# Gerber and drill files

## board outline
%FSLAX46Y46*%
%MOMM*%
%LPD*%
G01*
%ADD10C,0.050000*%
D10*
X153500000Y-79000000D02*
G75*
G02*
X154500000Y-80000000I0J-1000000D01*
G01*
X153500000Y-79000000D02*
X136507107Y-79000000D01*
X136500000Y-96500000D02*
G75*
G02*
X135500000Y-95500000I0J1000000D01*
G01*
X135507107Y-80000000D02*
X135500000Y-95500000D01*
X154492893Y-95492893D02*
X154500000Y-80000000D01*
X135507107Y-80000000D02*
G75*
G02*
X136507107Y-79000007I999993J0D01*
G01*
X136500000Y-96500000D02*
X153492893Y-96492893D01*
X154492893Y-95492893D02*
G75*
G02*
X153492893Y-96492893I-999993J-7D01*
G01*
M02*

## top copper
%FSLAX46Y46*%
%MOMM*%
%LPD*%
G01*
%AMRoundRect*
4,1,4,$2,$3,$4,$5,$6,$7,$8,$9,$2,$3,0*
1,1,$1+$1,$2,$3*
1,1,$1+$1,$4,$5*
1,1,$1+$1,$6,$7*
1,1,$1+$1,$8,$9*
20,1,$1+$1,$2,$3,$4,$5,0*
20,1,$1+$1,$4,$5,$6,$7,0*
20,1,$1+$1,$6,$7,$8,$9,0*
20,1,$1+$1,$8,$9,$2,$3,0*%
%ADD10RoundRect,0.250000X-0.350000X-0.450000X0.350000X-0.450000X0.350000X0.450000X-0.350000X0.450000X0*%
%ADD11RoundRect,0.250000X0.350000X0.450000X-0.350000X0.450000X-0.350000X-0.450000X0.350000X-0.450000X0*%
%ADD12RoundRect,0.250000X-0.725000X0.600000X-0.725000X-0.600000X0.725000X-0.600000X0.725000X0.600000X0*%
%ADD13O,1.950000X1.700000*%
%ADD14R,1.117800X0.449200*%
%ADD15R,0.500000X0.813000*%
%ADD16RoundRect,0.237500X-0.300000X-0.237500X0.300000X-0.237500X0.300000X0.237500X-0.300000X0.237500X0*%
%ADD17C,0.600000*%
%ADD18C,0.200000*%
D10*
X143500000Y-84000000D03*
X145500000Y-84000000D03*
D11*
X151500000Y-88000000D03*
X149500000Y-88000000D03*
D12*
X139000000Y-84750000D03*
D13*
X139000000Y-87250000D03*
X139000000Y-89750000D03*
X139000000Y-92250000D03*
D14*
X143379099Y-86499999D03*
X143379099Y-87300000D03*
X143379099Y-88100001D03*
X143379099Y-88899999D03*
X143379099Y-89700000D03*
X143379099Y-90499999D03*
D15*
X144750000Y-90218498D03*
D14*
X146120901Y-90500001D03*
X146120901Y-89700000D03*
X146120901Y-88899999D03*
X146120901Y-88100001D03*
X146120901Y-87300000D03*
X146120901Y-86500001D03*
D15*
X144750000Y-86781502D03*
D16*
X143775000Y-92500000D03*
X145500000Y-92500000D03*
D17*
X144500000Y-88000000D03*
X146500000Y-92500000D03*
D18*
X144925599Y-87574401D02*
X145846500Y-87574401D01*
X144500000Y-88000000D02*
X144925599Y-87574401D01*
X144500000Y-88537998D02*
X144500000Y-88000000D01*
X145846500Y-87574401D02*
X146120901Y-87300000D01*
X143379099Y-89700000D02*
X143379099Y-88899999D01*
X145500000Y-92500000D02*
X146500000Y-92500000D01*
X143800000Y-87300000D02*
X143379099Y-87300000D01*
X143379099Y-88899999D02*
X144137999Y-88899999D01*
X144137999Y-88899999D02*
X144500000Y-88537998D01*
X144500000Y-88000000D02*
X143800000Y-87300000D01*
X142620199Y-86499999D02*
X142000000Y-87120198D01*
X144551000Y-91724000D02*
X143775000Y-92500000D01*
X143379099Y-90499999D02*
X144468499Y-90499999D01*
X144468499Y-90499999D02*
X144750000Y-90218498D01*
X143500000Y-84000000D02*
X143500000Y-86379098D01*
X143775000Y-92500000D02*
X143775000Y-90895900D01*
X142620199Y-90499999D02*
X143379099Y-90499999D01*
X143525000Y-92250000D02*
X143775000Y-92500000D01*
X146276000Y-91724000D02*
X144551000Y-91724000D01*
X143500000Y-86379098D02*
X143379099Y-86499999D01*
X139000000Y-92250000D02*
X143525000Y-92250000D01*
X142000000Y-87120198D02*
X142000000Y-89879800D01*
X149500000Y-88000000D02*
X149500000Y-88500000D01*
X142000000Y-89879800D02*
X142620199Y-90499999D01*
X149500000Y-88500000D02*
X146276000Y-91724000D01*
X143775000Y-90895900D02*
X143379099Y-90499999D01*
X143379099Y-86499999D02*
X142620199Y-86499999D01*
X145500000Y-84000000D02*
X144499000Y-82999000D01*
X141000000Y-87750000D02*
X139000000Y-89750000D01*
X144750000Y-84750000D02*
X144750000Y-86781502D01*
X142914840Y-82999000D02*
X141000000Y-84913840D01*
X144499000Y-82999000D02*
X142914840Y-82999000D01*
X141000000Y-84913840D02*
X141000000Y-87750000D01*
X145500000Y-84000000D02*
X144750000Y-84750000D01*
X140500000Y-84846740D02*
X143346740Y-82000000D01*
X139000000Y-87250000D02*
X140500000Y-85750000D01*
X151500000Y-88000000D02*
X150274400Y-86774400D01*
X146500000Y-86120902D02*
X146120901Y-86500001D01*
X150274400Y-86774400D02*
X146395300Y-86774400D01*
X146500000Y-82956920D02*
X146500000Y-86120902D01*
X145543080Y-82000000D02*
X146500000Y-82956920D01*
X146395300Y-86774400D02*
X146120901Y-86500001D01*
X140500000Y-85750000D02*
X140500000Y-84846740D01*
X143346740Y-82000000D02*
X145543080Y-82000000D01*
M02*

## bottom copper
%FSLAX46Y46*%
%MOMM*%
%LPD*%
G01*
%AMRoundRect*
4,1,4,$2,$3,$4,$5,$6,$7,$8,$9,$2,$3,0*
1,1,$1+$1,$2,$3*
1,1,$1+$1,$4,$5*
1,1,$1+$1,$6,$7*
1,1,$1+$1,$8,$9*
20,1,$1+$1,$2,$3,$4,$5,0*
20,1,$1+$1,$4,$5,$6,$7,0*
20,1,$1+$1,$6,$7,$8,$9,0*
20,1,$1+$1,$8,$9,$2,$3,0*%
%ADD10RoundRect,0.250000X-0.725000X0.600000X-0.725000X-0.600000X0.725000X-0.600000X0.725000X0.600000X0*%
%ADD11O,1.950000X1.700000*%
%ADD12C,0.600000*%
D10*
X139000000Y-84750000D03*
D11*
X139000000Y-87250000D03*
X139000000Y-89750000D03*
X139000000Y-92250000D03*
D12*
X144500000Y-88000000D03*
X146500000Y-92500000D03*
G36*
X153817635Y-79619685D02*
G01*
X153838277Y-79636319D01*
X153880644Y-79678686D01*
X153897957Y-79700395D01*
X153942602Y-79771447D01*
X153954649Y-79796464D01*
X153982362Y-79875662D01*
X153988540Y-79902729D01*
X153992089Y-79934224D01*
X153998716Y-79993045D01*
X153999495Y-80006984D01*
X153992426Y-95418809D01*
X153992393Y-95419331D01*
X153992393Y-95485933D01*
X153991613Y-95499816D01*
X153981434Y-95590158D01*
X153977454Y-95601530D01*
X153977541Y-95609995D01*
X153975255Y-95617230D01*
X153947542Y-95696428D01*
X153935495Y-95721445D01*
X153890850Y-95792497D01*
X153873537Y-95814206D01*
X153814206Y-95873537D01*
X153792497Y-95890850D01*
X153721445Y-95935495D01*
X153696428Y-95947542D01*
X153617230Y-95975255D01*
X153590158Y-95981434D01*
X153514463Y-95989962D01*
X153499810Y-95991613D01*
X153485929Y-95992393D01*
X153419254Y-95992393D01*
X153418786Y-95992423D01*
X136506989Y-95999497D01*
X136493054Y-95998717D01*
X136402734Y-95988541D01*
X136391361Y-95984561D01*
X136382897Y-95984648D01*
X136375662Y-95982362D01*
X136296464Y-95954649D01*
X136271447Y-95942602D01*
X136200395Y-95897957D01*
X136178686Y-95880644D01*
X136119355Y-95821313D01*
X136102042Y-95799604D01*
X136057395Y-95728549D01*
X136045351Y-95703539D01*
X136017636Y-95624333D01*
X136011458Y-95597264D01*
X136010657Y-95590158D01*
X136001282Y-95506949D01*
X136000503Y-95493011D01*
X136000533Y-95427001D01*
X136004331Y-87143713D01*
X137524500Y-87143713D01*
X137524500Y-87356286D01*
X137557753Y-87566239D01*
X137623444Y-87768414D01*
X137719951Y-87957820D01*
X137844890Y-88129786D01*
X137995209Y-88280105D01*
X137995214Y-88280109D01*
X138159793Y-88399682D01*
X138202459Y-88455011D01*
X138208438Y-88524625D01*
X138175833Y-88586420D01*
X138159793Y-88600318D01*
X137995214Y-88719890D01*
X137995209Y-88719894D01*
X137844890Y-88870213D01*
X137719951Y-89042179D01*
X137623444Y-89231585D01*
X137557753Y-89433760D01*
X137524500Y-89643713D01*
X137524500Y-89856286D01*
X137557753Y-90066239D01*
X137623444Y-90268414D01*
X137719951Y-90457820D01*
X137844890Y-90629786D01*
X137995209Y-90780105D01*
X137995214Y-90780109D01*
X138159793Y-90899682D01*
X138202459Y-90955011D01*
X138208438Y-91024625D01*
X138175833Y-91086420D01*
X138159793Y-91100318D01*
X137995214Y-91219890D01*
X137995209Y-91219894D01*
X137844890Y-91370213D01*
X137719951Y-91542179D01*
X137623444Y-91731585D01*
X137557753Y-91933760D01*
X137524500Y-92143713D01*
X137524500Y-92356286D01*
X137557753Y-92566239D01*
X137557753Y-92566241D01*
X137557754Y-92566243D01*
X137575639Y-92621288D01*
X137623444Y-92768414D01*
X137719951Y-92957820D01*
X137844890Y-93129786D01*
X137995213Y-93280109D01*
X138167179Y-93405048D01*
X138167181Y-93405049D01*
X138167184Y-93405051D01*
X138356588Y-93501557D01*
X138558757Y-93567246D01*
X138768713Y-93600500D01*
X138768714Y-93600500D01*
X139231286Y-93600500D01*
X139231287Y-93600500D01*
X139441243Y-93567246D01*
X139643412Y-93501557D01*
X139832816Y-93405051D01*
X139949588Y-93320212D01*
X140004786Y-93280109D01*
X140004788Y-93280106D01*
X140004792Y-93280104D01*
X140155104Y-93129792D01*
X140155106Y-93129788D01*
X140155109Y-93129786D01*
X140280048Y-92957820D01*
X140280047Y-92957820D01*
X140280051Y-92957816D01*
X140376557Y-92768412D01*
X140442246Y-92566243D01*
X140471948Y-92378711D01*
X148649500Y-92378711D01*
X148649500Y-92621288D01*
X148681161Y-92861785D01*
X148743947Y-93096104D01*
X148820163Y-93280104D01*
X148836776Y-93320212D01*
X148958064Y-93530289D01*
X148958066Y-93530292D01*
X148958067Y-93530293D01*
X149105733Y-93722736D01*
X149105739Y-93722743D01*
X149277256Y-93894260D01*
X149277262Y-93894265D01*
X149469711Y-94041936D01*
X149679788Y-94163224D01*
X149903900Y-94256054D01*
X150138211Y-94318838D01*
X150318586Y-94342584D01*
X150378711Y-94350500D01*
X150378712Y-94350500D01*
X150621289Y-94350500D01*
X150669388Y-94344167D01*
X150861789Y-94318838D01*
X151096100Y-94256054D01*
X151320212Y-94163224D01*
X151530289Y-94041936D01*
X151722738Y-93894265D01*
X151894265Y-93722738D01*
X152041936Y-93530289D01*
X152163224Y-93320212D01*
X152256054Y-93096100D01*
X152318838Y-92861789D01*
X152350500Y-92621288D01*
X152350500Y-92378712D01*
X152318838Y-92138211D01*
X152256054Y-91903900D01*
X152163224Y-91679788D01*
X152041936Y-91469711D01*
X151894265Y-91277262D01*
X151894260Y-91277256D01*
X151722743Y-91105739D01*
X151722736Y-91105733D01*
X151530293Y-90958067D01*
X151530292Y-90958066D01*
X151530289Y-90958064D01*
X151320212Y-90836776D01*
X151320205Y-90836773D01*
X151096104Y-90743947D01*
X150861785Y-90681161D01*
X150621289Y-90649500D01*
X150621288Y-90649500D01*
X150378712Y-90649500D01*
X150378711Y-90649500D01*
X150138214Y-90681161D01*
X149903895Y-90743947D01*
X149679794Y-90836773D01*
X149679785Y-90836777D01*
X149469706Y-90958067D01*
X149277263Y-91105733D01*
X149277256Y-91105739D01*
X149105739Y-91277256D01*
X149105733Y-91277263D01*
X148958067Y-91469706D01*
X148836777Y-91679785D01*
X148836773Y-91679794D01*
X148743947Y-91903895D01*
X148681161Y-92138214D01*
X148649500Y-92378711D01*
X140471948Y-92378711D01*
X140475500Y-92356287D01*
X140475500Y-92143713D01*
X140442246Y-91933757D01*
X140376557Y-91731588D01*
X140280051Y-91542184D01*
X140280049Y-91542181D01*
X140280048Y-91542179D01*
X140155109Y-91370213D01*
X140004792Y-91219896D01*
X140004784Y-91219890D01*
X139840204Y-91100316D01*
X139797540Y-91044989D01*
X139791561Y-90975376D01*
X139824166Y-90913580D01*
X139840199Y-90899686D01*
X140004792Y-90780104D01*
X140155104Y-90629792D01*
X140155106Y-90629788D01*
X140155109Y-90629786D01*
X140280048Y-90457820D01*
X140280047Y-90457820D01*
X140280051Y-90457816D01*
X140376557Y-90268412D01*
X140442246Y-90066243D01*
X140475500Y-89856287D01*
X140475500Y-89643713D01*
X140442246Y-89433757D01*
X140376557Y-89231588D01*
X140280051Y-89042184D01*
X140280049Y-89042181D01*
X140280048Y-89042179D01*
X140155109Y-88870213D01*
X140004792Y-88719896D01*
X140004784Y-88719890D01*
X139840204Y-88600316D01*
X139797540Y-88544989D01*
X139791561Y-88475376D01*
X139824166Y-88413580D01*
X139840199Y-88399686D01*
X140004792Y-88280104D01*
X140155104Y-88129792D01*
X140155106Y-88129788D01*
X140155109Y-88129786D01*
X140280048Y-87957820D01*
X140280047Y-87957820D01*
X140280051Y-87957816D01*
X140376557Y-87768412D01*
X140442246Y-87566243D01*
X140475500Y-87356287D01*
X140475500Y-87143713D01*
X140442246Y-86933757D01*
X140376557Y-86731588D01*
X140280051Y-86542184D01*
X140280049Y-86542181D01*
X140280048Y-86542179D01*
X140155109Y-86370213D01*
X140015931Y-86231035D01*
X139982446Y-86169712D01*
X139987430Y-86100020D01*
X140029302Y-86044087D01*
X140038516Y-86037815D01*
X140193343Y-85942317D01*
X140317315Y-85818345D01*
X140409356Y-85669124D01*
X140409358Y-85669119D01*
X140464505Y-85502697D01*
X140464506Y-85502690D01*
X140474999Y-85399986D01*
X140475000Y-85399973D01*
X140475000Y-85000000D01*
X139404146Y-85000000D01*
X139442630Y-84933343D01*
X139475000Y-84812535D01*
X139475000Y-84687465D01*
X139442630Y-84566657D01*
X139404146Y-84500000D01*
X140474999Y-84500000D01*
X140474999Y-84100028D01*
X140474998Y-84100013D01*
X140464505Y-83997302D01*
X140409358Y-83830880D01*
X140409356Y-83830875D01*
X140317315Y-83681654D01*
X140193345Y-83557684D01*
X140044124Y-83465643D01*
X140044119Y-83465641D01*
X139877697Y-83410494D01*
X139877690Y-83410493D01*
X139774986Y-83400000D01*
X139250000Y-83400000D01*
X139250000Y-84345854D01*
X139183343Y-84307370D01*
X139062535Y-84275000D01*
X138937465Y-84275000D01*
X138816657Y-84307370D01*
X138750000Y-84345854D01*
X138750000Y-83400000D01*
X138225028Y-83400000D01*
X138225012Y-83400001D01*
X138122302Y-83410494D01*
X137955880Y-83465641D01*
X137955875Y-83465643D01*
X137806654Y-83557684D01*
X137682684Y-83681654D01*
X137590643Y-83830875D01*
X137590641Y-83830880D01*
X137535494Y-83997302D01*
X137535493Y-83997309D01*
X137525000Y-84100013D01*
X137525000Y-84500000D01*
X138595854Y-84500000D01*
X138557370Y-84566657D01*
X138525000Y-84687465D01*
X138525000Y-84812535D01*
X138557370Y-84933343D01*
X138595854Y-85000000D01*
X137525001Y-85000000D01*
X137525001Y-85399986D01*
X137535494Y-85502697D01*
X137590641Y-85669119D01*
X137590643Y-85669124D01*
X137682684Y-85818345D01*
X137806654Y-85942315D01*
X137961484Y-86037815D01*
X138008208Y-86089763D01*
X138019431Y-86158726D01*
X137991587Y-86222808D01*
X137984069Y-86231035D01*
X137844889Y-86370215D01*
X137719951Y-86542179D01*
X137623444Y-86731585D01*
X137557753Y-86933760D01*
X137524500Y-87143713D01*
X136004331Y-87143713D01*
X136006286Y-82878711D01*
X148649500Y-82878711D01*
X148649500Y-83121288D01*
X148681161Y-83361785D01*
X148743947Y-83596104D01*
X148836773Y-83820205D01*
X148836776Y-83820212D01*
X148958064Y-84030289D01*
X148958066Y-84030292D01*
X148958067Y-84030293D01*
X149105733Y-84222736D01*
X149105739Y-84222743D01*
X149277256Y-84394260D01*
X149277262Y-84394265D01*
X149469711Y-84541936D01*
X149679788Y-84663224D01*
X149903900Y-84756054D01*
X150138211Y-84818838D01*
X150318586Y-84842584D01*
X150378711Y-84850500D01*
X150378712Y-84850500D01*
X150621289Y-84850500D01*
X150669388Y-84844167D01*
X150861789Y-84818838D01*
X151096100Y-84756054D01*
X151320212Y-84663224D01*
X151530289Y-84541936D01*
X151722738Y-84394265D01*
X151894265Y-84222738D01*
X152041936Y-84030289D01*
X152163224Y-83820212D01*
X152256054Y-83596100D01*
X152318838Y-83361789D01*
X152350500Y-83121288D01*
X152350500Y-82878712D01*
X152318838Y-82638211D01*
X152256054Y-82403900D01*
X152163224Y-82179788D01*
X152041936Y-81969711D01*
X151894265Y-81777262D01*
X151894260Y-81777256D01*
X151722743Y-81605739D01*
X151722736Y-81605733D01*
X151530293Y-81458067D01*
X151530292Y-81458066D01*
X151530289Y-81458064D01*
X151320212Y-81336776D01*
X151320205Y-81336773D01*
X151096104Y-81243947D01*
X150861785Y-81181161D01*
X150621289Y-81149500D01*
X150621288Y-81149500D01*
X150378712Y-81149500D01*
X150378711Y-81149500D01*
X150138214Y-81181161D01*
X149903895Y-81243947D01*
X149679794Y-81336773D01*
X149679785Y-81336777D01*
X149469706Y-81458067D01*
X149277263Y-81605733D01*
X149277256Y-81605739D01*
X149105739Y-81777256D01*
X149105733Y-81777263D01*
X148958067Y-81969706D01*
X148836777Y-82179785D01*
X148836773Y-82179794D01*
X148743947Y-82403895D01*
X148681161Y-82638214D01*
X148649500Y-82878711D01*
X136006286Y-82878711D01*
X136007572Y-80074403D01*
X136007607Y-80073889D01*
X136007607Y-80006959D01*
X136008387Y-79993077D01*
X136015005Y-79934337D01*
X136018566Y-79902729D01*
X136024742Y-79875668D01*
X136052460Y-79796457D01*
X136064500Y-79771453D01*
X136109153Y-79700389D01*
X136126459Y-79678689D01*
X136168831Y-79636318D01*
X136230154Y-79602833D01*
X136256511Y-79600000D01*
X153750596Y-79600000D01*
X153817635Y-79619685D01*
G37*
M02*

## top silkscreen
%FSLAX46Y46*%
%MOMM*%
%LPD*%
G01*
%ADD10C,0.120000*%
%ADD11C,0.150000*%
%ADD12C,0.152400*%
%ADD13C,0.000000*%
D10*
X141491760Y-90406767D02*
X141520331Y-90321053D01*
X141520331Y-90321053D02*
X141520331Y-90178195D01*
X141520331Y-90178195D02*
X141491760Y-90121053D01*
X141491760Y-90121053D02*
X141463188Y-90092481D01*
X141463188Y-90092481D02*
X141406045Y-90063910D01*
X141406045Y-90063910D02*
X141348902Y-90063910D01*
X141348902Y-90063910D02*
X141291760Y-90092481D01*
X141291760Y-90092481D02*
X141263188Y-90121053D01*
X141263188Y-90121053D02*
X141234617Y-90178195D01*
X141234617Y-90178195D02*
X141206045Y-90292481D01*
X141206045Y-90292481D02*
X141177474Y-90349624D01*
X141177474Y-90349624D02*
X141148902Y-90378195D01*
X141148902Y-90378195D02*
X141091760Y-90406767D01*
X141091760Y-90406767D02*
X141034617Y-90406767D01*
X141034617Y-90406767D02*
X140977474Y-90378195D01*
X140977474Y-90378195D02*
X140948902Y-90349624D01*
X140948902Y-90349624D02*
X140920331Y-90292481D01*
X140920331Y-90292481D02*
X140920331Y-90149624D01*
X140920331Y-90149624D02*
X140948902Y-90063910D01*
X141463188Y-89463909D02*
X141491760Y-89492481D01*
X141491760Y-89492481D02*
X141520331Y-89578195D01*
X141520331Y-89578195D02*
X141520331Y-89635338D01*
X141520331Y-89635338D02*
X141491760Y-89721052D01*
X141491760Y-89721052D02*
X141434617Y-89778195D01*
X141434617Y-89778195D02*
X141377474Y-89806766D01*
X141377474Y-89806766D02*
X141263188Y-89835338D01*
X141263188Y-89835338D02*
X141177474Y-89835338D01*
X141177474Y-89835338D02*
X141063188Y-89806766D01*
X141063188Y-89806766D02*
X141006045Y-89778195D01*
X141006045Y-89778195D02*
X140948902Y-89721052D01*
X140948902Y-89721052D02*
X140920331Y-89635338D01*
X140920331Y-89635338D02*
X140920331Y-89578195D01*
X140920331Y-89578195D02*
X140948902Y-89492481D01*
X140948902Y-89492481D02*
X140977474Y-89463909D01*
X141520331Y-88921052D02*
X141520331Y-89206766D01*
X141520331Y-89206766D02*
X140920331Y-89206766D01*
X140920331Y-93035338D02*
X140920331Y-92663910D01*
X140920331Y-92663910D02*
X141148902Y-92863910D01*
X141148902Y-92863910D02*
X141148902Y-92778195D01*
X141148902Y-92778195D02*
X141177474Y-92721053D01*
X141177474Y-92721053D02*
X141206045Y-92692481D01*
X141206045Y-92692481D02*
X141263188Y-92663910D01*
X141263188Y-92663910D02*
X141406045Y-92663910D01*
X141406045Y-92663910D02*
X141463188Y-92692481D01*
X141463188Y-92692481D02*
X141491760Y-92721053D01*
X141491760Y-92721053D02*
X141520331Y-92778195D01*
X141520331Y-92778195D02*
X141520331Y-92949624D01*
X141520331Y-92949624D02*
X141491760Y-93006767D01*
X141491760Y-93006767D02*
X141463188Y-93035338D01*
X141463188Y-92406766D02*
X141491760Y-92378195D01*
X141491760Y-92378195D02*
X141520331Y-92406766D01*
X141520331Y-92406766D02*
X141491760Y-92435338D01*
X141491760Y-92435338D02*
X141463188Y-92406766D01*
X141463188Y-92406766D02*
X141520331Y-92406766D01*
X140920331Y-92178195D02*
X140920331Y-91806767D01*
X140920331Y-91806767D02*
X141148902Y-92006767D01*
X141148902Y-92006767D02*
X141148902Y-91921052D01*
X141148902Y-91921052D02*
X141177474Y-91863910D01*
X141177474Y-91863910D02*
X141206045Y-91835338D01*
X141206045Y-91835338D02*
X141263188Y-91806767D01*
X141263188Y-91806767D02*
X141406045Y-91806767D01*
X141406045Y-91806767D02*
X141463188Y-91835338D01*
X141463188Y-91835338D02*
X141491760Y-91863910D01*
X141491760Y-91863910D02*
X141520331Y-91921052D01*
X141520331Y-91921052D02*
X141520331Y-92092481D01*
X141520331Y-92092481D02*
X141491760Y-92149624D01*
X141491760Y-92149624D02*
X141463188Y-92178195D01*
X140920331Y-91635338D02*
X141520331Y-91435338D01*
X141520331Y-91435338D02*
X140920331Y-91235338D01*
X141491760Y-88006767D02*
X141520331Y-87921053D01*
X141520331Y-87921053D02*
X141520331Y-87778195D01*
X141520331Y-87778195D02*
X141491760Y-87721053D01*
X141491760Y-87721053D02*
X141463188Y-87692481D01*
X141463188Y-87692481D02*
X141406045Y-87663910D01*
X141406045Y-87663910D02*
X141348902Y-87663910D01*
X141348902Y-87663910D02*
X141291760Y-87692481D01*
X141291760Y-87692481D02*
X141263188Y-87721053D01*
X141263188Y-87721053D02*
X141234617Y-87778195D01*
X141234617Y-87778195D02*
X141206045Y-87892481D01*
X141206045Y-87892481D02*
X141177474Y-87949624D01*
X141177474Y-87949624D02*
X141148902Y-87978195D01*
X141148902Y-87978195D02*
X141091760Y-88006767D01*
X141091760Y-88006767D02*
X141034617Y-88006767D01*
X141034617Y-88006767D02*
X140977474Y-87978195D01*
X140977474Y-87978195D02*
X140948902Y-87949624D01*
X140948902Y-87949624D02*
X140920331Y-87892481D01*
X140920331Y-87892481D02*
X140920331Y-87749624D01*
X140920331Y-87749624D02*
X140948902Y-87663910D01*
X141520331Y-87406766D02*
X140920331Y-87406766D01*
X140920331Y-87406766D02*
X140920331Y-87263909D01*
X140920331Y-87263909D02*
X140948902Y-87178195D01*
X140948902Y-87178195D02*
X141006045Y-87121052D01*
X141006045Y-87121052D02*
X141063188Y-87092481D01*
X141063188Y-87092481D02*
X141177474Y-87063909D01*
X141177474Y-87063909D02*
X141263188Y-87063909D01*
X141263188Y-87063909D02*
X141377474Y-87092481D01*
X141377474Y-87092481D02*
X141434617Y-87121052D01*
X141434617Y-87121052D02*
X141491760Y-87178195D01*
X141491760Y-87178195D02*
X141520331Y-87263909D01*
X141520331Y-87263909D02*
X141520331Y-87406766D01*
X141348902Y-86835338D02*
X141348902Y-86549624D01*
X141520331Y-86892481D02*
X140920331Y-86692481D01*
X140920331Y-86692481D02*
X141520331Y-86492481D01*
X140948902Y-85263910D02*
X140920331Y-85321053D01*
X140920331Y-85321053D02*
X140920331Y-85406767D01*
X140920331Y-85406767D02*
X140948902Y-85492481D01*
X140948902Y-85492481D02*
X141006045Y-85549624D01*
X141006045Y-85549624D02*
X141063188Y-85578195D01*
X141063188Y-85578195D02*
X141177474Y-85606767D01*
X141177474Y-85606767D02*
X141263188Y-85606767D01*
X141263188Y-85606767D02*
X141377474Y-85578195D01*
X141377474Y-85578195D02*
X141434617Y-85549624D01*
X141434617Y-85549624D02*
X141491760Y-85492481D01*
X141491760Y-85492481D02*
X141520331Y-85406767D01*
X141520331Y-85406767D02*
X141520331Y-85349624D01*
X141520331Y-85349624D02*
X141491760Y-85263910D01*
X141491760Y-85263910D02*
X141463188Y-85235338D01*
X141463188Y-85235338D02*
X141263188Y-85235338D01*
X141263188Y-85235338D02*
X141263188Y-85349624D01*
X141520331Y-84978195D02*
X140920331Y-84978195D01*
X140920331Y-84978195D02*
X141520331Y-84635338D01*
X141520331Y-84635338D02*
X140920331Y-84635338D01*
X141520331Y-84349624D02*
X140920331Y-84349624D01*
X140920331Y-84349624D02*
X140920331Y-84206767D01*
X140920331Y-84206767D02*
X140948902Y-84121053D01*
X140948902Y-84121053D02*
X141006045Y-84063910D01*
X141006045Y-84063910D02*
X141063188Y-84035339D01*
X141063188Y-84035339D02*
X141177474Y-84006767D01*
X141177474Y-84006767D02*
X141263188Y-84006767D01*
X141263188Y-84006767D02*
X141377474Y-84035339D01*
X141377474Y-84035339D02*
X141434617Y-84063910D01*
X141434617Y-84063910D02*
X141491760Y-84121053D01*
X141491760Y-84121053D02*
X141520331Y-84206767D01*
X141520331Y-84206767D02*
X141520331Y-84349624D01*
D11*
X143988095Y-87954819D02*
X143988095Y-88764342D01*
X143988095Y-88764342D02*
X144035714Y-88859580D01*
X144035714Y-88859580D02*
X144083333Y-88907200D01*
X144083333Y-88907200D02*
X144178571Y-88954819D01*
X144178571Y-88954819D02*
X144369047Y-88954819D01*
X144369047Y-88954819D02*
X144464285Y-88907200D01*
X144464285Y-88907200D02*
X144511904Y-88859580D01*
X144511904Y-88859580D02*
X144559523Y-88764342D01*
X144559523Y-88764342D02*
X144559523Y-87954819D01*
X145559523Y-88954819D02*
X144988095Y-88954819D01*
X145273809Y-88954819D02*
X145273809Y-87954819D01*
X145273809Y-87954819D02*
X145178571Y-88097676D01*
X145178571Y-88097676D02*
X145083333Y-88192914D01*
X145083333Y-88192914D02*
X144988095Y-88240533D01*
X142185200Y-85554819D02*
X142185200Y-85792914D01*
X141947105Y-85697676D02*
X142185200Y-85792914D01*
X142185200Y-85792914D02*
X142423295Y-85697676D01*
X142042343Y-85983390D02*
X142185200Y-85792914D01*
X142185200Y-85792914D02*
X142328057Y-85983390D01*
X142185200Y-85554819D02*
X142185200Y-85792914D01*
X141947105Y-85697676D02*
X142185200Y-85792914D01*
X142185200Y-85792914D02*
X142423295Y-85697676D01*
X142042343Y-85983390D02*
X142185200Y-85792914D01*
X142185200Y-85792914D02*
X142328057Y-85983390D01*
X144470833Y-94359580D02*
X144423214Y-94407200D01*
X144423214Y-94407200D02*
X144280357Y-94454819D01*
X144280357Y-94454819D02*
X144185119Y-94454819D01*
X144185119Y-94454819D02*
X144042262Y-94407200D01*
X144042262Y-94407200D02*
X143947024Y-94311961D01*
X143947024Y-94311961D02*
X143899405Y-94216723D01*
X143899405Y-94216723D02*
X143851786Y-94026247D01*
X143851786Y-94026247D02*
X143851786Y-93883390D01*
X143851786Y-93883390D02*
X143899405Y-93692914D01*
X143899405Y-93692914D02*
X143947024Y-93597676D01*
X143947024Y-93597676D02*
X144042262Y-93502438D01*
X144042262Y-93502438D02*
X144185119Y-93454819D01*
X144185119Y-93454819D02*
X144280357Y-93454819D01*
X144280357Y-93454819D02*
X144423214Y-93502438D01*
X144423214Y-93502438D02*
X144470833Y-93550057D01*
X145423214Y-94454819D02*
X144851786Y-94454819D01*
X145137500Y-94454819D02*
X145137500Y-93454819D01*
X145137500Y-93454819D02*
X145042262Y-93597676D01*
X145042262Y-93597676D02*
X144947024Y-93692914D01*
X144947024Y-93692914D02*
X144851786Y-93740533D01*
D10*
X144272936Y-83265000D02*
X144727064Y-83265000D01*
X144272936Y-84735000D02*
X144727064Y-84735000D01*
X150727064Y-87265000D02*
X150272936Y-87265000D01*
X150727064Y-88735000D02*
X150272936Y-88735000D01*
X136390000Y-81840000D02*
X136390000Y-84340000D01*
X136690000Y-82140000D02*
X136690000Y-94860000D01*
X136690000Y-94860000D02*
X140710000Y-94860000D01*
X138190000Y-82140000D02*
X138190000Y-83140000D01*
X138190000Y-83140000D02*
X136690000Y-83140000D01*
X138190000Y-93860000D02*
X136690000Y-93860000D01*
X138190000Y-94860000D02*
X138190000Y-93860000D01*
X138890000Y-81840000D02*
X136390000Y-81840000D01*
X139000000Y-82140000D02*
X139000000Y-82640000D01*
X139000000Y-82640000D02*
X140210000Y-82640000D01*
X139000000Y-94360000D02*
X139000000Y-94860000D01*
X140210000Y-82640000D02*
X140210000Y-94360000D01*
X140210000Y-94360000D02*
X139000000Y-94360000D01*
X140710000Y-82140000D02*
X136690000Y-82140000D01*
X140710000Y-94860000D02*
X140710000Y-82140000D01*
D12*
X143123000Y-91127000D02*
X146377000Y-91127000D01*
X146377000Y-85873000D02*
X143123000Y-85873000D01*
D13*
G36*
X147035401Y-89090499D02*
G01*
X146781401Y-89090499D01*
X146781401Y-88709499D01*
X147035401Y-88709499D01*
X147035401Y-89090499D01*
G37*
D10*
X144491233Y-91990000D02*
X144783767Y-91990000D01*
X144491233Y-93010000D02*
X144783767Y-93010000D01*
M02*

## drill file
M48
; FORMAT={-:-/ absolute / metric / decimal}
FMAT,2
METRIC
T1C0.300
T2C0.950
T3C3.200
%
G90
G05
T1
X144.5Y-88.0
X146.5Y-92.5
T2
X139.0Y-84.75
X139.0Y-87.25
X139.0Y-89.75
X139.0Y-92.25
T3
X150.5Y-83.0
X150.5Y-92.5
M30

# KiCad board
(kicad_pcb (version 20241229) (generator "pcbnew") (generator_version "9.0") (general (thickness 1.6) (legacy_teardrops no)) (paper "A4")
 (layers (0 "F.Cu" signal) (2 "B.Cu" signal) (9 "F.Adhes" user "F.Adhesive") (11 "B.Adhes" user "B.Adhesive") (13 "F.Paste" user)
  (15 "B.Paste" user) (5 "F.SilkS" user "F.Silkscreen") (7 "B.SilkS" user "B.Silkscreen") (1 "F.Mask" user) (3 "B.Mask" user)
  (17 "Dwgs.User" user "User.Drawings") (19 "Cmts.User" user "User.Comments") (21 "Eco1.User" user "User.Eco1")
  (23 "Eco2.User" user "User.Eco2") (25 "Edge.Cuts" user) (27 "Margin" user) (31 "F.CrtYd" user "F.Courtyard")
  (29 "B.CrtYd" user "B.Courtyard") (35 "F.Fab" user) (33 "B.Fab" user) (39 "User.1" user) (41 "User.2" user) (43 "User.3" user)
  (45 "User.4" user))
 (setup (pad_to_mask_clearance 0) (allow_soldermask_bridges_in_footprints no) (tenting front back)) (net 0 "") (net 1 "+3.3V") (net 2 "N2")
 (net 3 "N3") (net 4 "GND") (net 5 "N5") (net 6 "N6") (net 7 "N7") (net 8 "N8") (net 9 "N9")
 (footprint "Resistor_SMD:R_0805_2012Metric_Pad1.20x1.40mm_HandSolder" (layer "F.Cu") (at 144.5 84)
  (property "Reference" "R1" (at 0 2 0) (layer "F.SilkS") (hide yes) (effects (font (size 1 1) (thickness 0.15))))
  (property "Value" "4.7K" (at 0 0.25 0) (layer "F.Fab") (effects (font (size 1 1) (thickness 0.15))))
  (fp_line (start -0.227064 -0.735) (end 0.227064 -0.735) (stroke (width 0.12) (type solid)) (layer "F.SilkS"))
  (fp_line (start -0.227064 0.735) (end 0.227064 0.735) (stroke (width 0.12) (type solid)) (layer "F.SilkS"))
  (pad "1" smd roundrect (at -1 0) (size 1.2 1.4) (layers "F.Cu" "F.Mask" "F.Paste") (roundrect_rratio 0.208333) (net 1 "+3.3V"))
  (pad "2" smd roundrect (at 1 0) (size 1.2 1.4) (layers "F.Cu" "F.Mask" "F.Paste") (roundrect_rratio 0.208333) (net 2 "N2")))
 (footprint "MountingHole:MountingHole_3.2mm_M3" (layer "F.Cu") (at 150.5 83)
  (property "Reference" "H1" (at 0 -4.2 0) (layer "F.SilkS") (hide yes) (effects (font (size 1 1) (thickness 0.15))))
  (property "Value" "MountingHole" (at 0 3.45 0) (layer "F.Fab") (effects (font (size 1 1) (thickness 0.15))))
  (pad "" np_thru_hole circle (at 0 0) (size 3.2 3.2) (drill 3.2) (layers "*.Cu" "*.Mask")))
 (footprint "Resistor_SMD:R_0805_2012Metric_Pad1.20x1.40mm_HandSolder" (layer "F.Cu") (at 150.5 88 180)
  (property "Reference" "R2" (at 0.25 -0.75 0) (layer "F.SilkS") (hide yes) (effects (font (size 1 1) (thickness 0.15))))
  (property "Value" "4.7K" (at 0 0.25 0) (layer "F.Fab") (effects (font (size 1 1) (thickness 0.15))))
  (fp_line (start -0.227064 0.735) (end 0.227064 0.735) (stroke (width 0.12) (type solid)) (layer "F.SilkS"))
  (fp_line (start -0.227064 -0.735) (end 0.227064 -0.735) (stroke (width 0.12) (type solid)) (layer "F.SilkS"))
  (pad "1" smd roundrect (at -1 0 180) (size 1.2 1.4) (layers "F.Cu" "F.Mask" "F.Paste") (roundrect_rratio 0.208333) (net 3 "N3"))
  (pad "2" smd roundrect (at 1 0 180) (size 1.2 1.4) (layers "F.Cu" "F.Mask" "F.Paste") (roundrect_rratio 0.208333) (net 1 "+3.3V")))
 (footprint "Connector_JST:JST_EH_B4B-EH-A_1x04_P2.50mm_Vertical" (layer "F.Cu") (at 139 84.75 -90)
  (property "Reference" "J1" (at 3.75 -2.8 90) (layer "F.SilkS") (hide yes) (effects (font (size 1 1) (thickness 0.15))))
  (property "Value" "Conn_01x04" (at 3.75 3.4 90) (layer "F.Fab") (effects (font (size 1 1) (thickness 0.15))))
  (fp_line (start -2.91 2.61) (end -0.41 2.61) (stroke (width 0.12) (type solid)) (layer "F.SilkS"))
  (fp_line (start -2.61 2.31) (end 10.11 2.31) (stroke (width 0.12) (type solid)) (layer "F.SilkS"))
  (fp_line (start 10.11 2.31) (end 10.11 -1.71) (stroke (width 0.12) (type solid)) (layer "F.SilkS"))
  (fp_line (start -2.61 0.81) (end -1.61 0.81) (stroke (width 0.12) (type solid)) (layer "F.SilkS"))
  (fp_line (start -1.61 0.81) (end -1.61 2.31) (stroke (width 0.12) (type solid)) (layer "F.SilkS"))
  (fp_line (start 9.11 0.81) (end 9.11 2.31) (stroke (width 0.12) (type solid)) (layer "F.SilkS"))
  (fp_line (start 10.11 0.81) (end 9.11 0.81) (stroke (width 0.12) (type solid)) (layer "F.SilkS"))
  (fp_line (start -2.91 0.11) (end -2.91 2.61) (stroke (width 0.12) (type solid)) (layer "F.SilkS"))
  (fp_line (start -2.61 0) (end -2.11 0) (stroke (width 0.12) (type solid)) (layer "F.SilkS"))
  (fp_line (start -2.11 0) (end -2.11 -1.21) (stroke (width 0.12) (type solid)) (layer "F.SilkS"))
  (fp_line (start 9.61 0) (end 10.11 0) (stroke (width 0.12) (type solid)) (layer "F.SilkS"))
  (fp_line (start -2.11 -1.21) (end 9.61 -1.21) (stroke (width 0.12) (type solid)) (layer "F.SilkS"))
  (fp_line (start 9.61 -1.21) (end 9.61 0) (stroke (width 0.12) (type solid)) (layer "F.SilkS"))
  (fp_line (start -2.61 -1.71) (end -2.61 2.31) (stroke (width 0.12) (type solid)) (layer "F.SilkS"))
  (fp_line (start 10.11 -1.71) (end -2.61 -1.71) (stroke (width 0.12) (type solid)) (layer "F.SilkS"))
  (pad "1" thru_hole roundrect (at 0 0 270) (size 1.7 1.95) (drill 0.95) (layers "*.Cu" "*.Mask") (remove_unused_layers no)
   (roundrect_rratio 0.147059) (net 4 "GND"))
  (pad "2" thru_hole oval (at 2.5 0 270) (size 1.7 1.95) (drill 0.95) (layers "*.Cu" "*.Mask") (remove_unused_layers no) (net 3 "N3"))
  (pad "3" thru_hole oval (at 5 0 270) (size 1.7 1.95) (drill 0.95) (layers "*.Cu" "*.Mask") (remove_unused_layers no) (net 2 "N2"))
  (pad "4" thru_hole oval (at 7.5 0 270) (size 1.7 1.95) (drill 0.95) (layers "*.Cu" "*.Mask") (remove_unused_layers no) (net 1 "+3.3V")))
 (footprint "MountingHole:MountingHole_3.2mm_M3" (layer "F.Cu") (at 150.5 92.5)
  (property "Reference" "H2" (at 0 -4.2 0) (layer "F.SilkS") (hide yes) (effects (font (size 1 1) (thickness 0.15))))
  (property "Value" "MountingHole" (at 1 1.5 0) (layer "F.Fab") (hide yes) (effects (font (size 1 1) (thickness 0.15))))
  (pad "" np_thru_hole circle (at 0 0) (size 3.2 3.2) (drill 3.2) (layers "*.Cu" "*.Mask")))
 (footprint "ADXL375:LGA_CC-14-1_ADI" (layer "F.Cu") (at 144.75 88.5)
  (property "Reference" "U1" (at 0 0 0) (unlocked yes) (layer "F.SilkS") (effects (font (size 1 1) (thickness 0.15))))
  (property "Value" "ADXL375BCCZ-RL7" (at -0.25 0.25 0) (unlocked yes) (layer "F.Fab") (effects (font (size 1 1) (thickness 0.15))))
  (fp_line (start -1.627 2.627) (end 1.627 2.627) (stroke (width 0.1524) (type solid)) (layer "F.SilkS"))
  (fp_line (start 1.627 -2.627) (end -1.627 -2.627) (stroke (width 0.1524) (type solid)) (layer "F.SilkS"))
  (fp_poly
   (pts (xy 2.285401 0.209499) (xy 2.285401 0.590499) (xy 2.031401 0.590499) (xy 2.031401 0.209499)) (stroke (width 0) (type solid))
   (fill yes) (layer "F.SilkS"))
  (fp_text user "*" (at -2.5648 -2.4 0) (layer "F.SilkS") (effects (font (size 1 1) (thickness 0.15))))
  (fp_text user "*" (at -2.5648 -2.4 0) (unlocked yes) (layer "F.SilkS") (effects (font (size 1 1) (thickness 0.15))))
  (pad "1" smd rect (at -1.370901 -2.000001 90) (size 0.4492 1.1178) (layers "F.Cu" "F.Mask" "F.Paste") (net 1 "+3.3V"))
  (pad "2" smd rect (at -1.370901 -1.2 90) (size 0.4492 1.1178) (layers "F.Cu" "F.Mask" "F.Paste") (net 4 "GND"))
  (pad "3" smd rect (at -1.370901 -0.399999 90) (size 0.4492 1.1178) (layers "F.Cu" "F.Mask" "F.Paste") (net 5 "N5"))
  (pad "4" smd rect (at -1.370901 0.399999 90) (size 0.4492 1.1178) (layers "F.Cu" "F.Mask" "F.Paste") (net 4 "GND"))
  (pad "5" smd rect (at -1.370901 1.2 90) (size 0.4492 1.1178) (layers "F.Cu" "F.Mask" "F.Paste") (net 4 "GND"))
  (pad "6" smd rect (at -1.370901 1.999999 90) (size 0.4492 1.1178) (layers "F.Cu" "F.Mask" "F.Paste") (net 1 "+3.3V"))
  (pad "7" smd rect (at 0 1.718498) (size 0.5 0.813) (layers "F.Cu" "F.Mask" "F.Paste") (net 1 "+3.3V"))
  (pad "8" smd rect (at 1.370901 2.000001 90) (size 0.4492 1.1178) (layers "F.Cu" "F.Mask" "F.Paste") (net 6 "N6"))
  (pad "9" smd rect (at 1.370901 1.2 90) (size 0.4492 1.1178) (layers "F.Cu" "F.Mask" "F.Paste") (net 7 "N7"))
  (pad "10" smd rect (at 1.370901 0.399999 90) (size 0.4492 1.1178) (layers "F.Cu" "F.Mask" "F.Paste") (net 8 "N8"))
  (pad "11" smd rect (at 1.370901 -0.399999 90) (size 0.4492 1.1178) (layers "F.Cu" "F.Mask" "F.Paste") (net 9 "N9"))
  (pad "12" smd rect (at 1.370901 -1.2 90) (size 0.4492 1.1178) (layers "F.Cu" "F.Mask" "F.Paste") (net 4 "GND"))
  (pad "13" smd rect (at 1.370901 -1.999999 90) (size 0.4492 1.1178) (layers "F.Cu" "F.Mask" "F.Paste") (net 3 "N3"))
  (pad "14" smd rect (at 0 -1.718498) (size 0.5 0.813) (layers "F.Cu" "F.Mask" "F.Paste") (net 2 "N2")))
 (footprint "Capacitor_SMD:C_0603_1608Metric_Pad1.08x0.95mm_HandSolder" (layer "F.Cu") (at 144.6375 92.5)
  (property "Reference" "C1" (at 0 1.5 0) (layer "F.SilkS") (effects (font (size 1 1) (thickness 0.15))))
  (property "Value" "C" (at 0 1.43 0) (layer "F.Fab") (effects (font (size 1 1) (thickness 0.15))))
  (fp_line (start -0.146267 -0.51) (end 0.146267 -0.51) (stroke (width 0.12) (type solid)) (layer "F.SilkS"))
  (fp_line (start -0.146267 0.51) (end 0.146267 0.51) (stroke (width 0.12) (type solid)) (layer "F.SilkS"))
  (pad "1" smd roundrect (at -0.8625 0) (size 1.075 0.95) (layers "F.Cu" "F.Mask" "F.Paste") (roundrect_rratio 0.25) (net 1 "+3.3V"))
  (pad "2" smd roundrect (at 0.8625 0) (size 1.075 0.95) (layers "F.Cu" "F.Mask" "F.Paste") (roundrect_rratio 0.25) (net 4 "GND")))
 (gr_arc (start 153.5 79) (mid 154.207107 79.292893) (end 154.5 80) (stroke (width 0.05) (type default)) (layer "Edge.Cuts"))
 (gr_line (start 153.5 79) (end 136.507107 79) (stroke (width 0.05) (type default)) (layer "Edge.Cuts"))
 (gr_arc (start 136.5 96.5) (mid 135.792893 96.207107) (end 135.5 95.5) (stroke (width 0.05) (type default)) (layer "Edge.Cuts"))
 (gr_line (start 135.507107 80) (end 135.5 95.5) (stroke (width 0.05) (type default)) (layer "Edge.Cuts"))
 (gr_line (start 154.492893 95.492893) (end 154.5 80) (stroke (width 0.05) (type default)) (layer "Edge.Cuts"))
 (gr_arc (start 135.507107 80) (mid 135.8 79.292893) (end 136.507107 79) (stroke (width 0.05) (type default)) (layer "Edge.Cuts"))
 (gr_line (start 136.5 96.5) (end 153.492893 96.492893) (stroke (width 0.05) (type default)) (layer "Edge.Cuts"))
 (gr_arc (start 154.492893 95.492893) (mid 154.2 96.2) (end 153.492893 96.492893) (stroke (width 0.05) (type default)) (layer "Edge.Cuts"))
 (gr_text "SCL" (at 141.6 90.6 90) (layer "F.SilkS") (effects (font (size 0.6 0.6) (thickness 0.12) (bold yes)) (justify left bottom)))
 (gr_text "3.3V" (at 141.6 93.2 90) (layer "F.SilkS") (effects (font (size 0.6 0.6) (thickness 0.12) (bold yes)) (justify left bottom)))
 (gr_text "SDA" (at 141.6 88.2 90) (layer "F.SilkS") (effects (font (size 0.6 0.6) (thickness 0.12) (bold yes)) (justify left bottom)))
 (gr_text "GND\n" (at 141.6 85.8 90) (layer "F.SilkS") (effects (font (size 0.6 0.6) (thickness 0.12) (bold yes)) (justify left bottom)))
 (segment (start 144.925599 87.574401) (end 145.8465 87.574401) (width 0.2) (layer "F.Cu") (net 4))
 (segment (start 144.5 88) (end 144.925599 87.574401) (width 0.2) (layer "F.Cu") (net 4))
 (segment (start 144.5 88.537998) (end 144.5 88) (width 0.2) (layer "F.Cu") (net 4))
 (segment (start 145.8465 87.574401) (end 146.120901 87.3) (width 0.2) (layer "F.Cu") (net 4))
 (segment (start 143.379099 89.7) (end 143.379099 88.899999) (width 0.2) (layer "F.Cu") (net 4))
 (segment (start 145.5 92.5) (end 146.5 92.5) (width 0.2) (layer "F.Cu") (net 4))
 (segment (start 143.8 87.3) (end 143.379099 87.3) (width 0.2) (layer "F.Cu") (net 4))
 (segment (start 143.379099 88.899999) (end 144.137999 88.899999) (width 0.2) (layer "F.Cu") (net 4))
 (segment (start 144.137999 88.899999) (end 144.5 88.537998) (width 0.2) (layer "F.Cu") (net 4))
 (segment (start 144.5 88) (end 143.8 87.3) (width 0.2) (layer "F.Cu") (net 4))
 (via (at 144.5 88) (size 0.6) (drill 0.3) (layers "F.Cu" "B.Cu") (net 4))
 (via (at 146.5 92.5) (size 0.6) (drill 0.3) (layers "F.Cu" "B.Cu") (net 4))
 (segment (start 142.620199 86.499999) (end 142 87.120198) (width 0.2) (layer "F.Cu") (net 1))
 (segment (start 144.551 91.724) (end 143.775 92.5) (width 0.2) (layer "F.Cu") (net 1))
 (segment (start 143.379099 90.499999) (end 144.468499 90.499999) (width 0.2) (layer "F.Cu") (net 1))
 (segment (start 144.468499 90.499999) (end 144.75 90.218498) (width 0.2) (layer "F.Cu") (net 1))
 (segment (start 143.5 84) (end 143.5 86.379098) (width 0.2) (layer "F.Cu") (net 1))
 (segment (start 143.775 92.5) (end 143.775 90.8959) (width 0.2) (layer "F.Cu") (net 1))
 (segment (start 142.620199 90.499999) (end 143.379099 90.499999) (width 0.2) (layer "F.Cu") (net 1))
 (segment (start 143.525 92.25) (end 143.775 92.5) (width 0.2) (layer "F.Cu") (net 1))
 (segment (start 146.276 91.724) (end 144.551 91.724) (width 0.2) (layer "F.Cu") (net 1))
 (segment (start 143.5 86.379098) (end 143.379099 86.499999) (width 0.2) (layer "F.Cu") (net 1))
 (segment (start 139 92.25) (end 143.525 92.25) (width 0.2) (layer "F.Cu") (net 1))
 (segment (start 142 87.120198) (end 142 89.8798) (width 0.2) (layer "F.Cu") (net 1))
 (segment (start 149.5 88) (end 149.5 88.5) (width 0.2) (layer "F.Cu") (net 1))
 (segment (start 142 89.8798) (end 142.620199 90.499999) (width 0.2) (layer "F.Cu") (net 1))
 (segment (start 149.5 88.5) (end 146.276 91.724) (width 0.2) (layer "F.Cu") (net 1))
 (segment (start 143.775 90.8959) (end 143.379099 90.499999) (width 0.2) (layer "F.Cu") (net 1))
 (segment (start 143.379099 86.499999) (end 142.620199 86.499999) (width 0.2) (layer "F.Cu") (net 1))
 (segment (start 145.5 84) (end 144.499 82.999) (width 0.2) (layer "F.Cu") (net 2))
 (segment (start 141 87.75) (end 139 89.75) (width 0.2) (layer "F.Cu") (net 2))
 (segment (start 144.75 84.75) (end 144.75 86.781502) (width 0.2) (layer "F.Cu") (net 2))
 (segment (start 142.91484 82.999) (end 141 84.91384) (width 0.2) (layer "F.Cu") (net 2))
 (segment (start 144.499 82.999) (end 142.91484 82.999) (width 0.2) (layer "F.Cu") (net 2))
 (segment (start 141 84.91384) (end 141 87.75) (width 0.2) (layer "F.Cu") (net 2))
 (segment (start 145.5 84) (end 144.75 84.75) (width 0.2) (layer "F.Cu") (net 2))
 (segment (start 140.5 84.84674) (end 143.34674 82) (width 0.2) (layer "F.Cu") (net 3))
 (segment (start 139 87.25) (end 140.5 85.75) (width 0.2) (layer "F.Cu") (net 3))
 (segment (start 151.5 88) (end 150.2744 86.7744) (width 0.2) (layer "F.Cu") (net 3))
 (segment (start 146.5 86.120902) (end 146.120901 86.500001) (width 0.2) (layer "F.Cu") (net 3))
 (segment (start 150.2744 86.7744) (end 146.3953 86.7744) (width 0.2) (layer "F.Cu") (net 3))
 (segment (start 146.5 82.95692) (end 146.5 86.120902) (width 0.2) (layer "F.Cu") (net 3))
 (segment (start 145.54308 82) (end 146.5 82.95692) (width 0.2) (layer "F.Cu") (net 3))
 (segment (start 146.3953 86.7744) (end 146.120901 86.500001) (width 0.2) (layer "F.Cu") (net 3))
 (segment (start 140.5 85.75) (end 140.5 84.84674) (width 0.2) (layer "F.Cu") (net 3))
 (segment (start 143.34674 82) (end 145.54308 82) (width 0.2) (layer "F.Cu") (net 3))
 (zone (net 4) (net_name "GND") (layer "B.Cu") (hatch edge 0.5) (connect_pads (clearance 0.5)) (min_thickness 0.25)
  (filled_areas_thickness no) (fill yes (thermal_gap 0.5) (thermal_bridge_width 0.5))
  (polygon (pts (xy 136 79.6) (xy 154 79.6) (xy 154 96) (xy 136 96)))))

